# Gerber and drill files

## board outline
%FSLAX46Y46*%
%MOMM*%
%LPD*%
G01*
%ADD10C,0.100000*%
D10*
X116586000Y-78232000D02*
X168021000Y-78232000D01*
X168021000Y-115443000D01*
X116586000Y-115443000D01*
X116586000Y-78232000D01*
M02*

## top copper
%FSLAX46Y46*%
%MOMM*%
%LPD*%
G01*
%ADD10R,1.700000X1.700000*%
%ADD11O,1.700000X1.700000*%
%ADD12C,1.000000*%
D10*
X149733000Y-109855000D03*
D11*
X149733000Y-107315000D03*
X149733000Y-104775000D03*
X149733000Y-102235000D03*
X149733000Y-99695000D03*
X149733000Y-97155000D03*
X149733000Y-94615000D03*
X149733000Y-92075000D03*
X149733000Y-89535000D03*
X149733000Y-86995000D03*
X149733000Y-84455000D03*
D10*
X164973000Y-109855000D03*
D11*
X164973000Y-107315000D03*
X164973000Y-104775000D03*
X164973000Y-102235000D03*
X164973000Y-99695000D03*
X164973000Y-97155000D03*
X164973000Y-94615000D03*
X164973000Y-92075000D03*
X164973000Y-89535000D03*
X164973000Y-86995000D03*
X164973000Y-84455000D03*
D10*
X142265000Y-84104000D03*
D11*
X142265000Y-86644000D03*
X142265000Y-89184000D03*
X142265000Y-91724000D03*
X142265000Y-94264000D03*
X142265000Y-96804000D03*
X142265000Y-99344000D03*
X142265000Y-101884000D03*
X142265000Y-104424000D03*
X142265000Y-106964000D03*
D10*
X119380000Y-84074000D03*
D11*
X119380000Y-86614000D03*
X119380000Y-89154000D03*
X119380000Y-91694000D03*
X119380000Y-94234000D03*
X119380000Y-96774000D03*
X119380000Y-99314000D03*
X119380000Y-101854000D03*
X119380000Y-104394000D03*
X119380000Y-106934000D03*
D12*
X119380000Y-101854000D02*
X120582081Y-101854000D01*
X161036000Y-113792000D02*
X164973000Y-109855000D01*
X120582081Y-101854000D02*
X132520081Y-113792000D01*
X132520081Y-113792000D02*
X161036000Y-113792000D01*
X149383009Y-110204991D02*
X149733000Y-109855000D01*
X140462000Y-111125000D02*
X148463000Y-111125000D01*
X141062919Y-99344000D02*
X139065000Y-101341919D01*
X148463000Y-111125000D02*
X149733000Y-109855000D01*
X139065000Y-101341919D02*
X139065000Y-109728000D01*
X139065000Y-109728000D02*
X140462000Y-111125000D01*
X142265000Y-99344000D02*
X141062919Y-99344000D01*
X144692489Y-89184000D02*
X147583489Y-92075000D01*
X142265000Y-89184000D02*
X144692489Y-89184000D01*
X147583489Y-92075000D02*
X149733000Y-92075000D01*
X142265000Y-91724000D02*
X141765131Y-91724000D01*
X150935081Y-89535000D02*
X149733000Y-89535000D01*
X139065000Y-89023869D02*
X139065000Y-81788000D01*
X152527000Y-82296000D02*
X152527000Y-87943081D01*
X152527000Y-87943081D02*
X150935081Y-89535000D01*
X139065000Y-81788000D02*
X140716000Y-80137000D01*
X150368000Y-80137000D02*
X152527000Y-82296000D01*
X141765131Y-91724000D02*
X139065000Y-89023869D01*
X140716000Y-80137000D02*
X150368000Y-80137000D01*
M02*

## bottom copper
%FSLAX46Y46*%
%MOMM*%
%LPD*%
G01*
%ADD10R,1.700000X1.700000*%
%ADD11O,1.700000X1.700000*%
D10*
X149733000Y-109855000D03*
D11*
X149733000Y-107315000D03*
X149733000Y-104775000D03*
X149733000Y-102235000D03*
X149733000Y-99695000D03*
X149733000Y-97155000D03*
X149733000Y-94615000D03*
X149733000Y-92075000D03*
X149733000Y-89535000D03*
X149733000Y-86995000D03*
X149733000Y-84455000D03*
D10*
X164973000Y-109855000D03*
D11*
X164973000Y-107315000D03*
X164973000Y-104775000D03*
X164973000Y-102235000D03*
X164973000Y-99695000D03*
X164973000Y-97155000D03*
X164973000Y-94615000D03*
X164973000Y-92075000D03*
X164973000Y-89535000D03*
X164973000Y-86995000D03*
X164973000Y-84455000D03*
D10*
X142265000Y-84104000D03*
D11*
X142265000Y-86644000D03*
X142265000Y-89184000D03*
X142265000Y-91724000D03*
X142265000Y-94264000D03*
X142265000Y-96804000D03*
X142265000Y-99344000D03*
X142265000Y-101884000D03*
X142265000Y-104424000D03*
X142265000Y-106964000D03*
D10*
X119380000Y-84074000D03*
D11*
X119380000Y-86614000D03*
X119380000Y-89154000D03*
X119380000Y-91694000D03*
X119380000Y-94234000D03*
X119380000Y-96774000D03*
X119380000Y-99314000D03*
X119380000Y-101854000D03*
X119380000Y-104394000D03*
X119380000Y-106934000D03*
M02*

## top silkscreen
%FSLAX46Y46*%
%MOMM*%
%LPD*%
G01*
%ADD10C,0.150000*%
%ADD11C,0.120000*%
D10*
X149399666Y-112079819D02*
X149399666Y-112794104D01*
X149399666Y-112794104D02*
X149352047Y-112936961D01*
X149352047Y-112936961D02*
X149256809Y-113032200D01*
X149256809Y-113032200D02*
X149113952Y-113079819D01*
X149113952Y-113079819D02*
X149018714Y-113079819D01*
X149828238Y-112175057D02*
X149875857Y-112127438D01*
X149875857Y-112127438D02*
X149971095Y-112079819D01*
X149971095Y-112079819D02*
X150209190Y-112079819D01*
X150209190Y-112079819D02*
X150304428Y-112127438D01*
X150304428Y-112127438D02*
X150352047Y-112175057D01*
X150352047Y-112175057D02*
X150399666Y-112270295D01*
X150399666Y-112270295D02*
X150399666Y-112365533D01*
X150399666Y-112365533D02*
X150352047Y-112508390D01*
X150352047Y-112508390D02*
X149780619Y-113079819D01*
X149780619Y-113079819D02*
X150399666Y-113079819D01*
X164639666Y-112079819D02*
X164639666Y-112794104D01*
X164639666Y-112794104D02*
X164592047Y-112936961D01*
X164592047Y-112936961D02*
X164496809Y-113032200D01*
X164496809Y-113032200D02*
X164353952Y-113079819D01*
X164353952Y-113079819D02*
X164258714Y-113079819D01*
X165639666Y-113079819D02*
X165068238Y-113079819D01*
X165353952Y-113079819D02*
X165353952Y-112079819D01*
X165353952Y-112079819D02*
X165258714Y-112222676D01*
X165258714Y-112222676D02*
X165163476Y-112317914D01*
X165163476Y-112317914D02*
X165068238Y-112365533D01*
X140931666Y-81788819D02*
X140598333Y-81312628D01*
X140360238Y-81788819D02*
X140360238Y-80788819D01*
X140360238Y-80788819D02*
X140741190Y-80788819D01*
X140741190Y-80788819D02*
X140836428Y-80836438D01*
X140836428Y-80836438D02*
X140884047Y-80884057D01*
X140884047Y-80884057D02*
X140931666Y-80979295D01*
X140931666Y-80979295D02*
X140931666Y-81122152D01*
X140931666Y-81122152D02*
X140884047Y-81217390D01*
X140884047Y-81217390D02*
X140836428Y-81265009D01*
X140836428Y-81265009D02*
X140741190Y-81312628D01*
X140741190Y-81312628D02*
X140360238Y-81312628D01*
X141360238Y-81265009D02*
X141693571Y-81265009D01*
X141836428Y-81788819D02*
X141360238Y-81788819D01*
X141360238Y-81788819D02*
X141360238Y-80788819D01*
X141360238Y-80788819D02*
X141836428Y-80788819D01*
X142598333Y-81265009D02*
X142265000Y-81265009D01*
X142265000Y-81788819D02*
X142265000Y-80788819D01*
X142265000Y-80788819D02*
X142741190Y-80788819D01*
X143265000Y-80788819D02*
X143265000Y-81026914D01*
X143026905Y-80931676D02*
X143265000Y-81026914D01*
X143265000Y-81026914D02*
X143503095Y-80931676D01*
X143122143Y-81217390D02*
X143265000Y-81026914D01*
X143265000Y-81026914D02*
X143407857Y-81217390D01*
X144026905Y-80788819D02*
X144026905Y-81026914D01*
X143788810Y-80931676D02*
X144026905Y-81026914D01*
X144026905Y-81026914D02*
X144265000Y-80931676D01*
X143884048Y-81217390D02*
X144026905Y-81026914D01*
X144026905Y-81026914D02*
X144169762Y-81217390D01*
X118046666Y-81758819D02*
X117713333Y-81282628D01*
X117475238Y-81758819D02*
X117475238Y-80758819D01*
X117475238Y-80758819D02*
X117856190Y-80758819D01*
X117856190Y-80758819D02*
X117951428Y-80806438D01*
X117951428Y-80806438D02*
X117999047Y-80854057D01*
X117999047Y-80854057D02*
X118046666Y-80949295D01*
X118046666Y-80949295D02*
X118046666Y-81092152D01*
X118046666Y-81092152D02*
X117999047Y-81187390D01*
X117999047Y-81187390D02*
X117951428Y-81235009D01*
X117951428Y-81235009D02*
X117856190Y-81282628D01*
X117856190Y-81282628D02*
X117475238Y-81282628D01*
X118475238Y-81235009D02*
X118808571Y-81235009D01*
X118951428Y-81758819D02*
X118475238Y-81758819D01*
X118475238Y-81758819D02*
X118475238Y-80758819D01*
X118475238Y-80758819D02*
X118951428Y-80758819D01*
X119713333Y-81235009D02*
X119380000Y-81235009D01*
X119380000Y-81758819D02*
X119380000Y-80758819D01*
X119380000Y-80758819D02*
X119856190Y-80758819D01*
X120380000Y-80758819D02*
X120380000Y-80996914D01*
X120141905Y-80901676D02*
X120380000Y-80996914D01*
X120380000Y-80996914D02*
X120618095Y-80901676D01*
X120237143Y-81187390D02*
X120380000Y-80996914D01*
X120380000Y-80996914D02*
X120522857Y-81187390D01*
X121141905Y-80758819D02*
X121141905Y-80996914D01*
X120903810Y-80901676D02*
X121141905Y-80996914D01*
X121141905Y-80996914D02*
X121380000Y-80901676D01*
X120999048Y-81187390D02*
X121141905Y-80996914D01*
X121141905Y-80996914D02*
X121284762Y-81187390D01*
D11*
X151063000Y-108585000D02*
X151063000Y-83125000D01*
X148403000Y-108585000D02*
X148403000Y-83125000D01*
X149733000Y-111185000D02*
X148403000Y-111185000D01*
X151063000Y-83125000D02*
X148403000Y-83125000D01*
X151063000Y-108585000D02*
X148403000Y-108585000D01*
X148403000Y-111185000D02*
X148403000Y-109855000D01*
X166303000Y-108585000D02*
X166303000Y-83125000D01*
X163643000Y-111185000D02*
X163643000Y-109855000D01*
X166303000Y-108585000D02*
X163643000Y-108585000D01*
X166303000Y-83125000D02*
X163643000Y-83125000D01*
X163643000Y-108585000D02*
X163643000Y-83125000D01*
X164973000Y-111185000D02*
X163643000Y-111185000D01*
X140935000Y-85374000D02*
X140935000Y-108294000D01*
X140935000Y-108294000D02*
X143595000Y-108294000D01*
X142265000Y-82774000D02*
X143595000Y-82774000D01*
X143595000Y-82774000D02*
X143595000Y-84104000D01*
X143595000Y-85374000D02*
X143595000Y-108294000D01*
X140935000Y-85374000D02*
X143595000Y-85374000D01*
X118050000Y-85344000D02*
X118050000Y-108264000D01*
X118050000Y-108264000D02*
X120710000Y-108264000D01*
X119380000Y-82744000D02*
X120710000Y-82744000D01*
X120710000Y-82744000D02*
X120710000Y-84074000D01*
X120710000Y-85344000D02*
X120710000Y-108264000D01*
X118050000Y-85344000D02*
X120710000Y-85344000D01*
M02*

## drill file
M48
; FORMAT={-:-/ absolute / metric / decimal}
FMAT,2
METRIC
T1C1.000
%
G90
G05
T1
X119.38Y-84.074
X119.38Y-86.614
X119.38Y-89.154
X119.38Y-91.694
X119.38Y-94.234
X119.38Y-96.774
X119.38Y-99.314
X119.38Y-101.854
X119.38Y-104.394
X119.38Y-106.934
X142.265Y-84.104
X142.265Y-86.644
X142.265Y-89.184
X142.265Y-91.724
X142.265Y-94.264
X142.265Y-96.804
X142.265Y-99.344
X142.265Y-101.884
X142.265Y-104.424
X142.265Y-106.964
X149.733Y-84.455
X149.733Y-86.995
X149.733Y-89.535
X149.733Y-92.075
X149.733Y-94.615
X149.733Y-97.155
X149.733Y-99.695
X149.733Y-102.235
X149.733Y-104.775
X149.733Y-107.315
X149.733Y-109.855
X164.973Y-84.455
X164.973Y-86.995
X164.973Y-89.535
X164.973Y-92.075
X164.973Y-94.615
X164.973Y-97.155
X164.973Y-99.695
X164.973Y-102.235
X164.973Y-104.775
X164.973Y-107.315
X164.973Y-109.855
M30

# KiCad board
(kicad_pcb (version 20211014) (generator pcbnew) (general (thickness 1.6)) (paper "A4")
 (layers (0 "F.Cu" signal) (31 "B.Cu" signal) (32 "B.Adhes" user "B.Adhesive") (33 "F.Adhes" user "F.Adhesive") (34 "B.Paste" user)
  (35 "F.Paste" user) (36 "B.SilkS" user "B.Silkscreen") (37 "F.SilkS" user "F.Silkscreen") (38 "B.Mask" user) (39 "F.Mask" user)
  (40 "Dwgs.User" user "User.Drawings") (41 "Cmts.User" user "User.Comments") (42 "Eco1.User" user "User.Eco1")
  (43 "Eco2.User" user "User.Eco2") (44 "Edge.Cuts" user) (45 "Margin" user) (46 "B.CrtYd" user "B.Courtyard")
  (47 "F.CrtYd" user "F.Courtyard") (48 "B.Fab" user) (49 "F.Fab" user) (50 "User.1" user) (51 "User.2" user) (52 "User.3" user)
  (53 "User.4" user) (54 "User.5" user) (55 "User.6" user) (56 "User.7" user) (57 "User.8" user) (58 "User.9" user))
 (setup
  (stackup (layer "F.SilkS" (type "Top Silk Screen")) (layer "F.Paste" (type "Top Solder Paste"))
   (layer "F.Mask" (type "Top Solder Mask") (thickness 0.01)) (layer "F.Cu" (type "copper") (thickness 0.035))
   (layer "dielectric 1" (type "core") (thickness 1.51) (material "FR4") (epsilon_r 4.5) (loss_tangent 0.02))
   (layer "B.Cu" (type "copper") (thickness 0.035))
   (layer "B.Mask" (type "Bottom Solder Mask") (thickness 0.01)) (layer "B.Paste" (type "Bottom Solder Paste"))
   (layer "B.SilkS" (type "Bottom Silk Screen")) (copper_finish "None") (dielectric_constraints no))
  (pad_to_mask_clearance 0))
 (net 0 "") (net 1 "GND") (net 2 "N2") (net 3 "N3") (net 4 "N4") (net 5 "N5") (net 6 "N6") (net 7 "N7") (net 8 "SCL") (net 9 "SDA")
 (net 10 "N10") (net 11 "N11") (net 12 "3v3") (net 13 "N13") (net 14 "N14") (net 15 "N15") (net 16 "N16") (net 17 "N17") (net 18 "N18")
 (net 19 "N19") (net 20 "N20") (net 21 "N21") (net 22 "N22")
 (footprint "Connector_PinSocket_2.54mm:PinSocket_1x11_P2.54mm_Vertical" (layer "F.Cu") (at 149.733 109.855 180)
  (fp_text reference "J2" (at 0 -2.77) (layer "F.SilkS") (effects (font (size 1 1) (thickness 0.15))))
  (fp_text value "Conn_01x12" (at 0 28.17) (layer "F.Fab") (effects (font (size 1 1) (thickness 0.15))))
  (fp_line (start -1.33 1.27) (end -1.33 26.73) (layer "F.SilkS") (width 0.12))
  (fp_line (start 1.33 1.27) (end 1.33 26.73) (layer "F.SilkS") (width 0.12))
  (fp_line (start 0 -1.33) (end 1.33 -1.33) (layer "F.SilkS") (width 0.12))
  (fp_line (start -1.33 26.73) (end 1.33 26.73) (layer "F.SilkS") (width 0.12))
  (fp_line (start -1.33 1.27) (end 1.33 1.27) (layer "F.SilkS") (width 0.12))
  (fp_line (start 1.33 -1.33) (end 1.33 0) (layer "F.SilkS") (width 0.12))
  (pad "1" thru_hole rect (at 0 0 180) (size 1.7 1.7) (drill 1) (layers *.Cu *.Mask) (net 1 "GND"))
  (pad "2" thru_hole oval (at 0 2.54 180) (size 1.7 1.7) (drill 1) (layers *.Cu *.Mask) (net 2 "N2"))
  (pad "3" thru_hole oval (at 0 5.08 180) (size 1.7 1.7) (drill 1) (layers *.Cu *.Mask) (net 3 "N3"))
  (pad "4" thru_hole oval (at 0 7.62 180) (size 1.7 1.7) (drill 1) (layers *.Cu *.Mask) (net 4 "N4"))
  (pad "5" thru_hole oval (at 0 10.16 180) (size 1.7 1.7) (drill 1) (layers *.Cu *.Mask) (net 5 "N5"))
  (pad "6" thru_hole oval (at 0 12.7 180) (size 1.7 1.7) (drill 1) (layers *.Cu *.Mask) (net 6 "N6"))
  (pad "7" thru_hole oval (at 0 15.24 180) (size 1.7 1.7) (drill 1) (layers *.Cu *.Mask) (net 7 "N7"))
  (pad "8" thru_hole oval (at 0 17.78 180) (size 1.7 1.7) (drill 1) (layers *.Cu *.Mask) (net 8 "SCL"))
  (pad "9" thru_hole oval (at 0 20.32 180) (size 1.7 1.7) (drill 1) (layers *.Cu *.Mask) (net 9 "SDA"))
  (pad "10" thru_hole oval (at 0 22.86 180) (size 1.7 1.7) (drill 1) (layers *.Cu *.Mask) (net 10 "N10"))
  (pad "11" thru_hole oval (at 0 25.4 180) (size 1.7 1.7) (drill 1) (layers *.Cu *.Mask) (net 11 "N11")))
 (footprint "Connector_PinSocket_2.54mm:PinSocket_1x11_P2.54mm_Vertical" (layer "F.Cu") (at 164.973 109.855 180)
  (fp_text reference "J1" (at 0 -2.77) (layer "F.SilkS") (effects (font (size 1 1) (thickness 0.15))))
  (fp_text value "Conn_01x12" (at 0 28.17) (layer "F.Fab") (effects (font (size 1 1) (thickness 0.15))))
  (fp_line (start -1.33 1.27) (end -1.33 26.73) (layer "F.SilkS") (width 0.12))
  (fp_line (start 1.33 -1.33) (end 1.33 0) (layer "F.SilkS") (width 0.12))
  (fp_line (start -1.33 1.27) (end 1.33 1.27) (layer "F.SilkS") (width 0.12))
  (fp_line (start -1.33 26.73) (end 1.33 26.73) (layer "F.SilkS") (width 0.12))
  (fp_line (start 1.33 1.27) (end 1.33 26.73) (layer "F.SilkS") (width 0.12))
  (fp_line (start 0 -1.33) (end 1.33 -1.33) (layer "F.SilkS") (width 0.12))
  (pad "1" thru_hole rect (at 0 0 180) (size 1.7 1.7) (drill 1) (layers *.Cu *.Mask) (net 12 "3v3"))
  (pad "2" thru_hole oval (at 0 2.54 180) (size 1.7 1.7) (drill 1) (layers *.Cu *.Mask) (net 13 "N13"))
  (pad "3" thru_hole oval (at 0 5.08 180) (size 1.7 1.7) (drill 1) (layers *.Cu *.Mask) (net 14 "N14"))
  (pad "4" thru_hole oval (at 0 7.62 180) (size 1.7 1.7) (drill 1) (layers *.Cu *.Mask) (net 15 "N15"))
  (pad "5" thru_hole oval (at 0 10.16 180) (size 1.7 1.7) (drill 1) (layers *.Cu *.Mask) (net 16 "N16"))
  (pad "6" thru_hole oval (at 0 12.7 180) (size 1.7 1.7) (drill 1) (layers *.Cu *.Mask) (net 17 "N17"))
  (pad "7" thru_hole oval (at 0 15.24 180) (size 1.7 1.7) (drill 1) (layers *.Cu *.Mask) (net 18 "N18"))
  (pad "8" thru_hole oval (at 0 17.78 180) (size 1.7 1.7) (drill 1) (layers *.Cu *.Mask) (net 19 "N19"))
  (pad "9" thru_hole oval (at 0 20.32 180) (size 1.7 1.7) (drill 1) (layers *.Cu *.Mask) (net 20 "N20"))
  (pad "10" thru_hole oval (at 0 22.86 180) (size 1.7 1.7) (drill 1) (layers *.Cu *.Mask) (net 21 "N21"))
  (pad "11" thru_hole oval (at 0 25.4 180) (size 1.7 1.7) (drill 1) (layers *.Cu *.Mask) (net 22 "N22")))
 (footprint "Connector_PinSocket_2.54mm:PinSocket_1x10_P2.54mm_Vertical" (layer "F.Cu") (at 142.265 84.104)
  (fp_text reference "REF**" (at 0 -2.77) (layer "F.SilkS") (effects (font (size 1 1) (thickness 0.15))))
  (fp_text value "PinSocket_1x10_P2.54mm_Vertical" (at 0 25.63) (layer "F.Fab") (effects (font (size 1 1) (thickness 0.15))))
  (fp_line (start -1.33 1.27) (end -1.33 24.19) (layer "F.SilkS") (width 0.12))
  (fp_line (start -1.33 24.19) (end 1.33 24.19) (layer "F.SilkS") (width 0.12))
  (fp_line (start 0 -1.33) (end 1.33 -1.33) (layer "F.SilkS") (width 0.12))
  (fp_line (start 1.33 -1.33) (end 1.33 0) (layer "F.SilkS") (width 0.12))
  (fp_line (start 1.33 1.27) (end 1.33 24.19) (layer "F.SilkS") (width 0.12))
  (fp_line (start -1.33 1.27) (end 1.33 1.27) (layer "F.SilkS") (width 0.12))
  (pad "1" thru_hole rect (at 0 0) (size 1.7 1.7) (drill 1) (layers *.Cu *.Mask))
  (pad "2" thru_hole oval (at 0 2.54) (size 1.7 1.7) (drill 1) (layers *.Cu *.Mask))
  (pad "3" thru_hole oval (at 0 5.08) (size 1.7 1.7) (drill 1) (layers *.Cu *.Mask) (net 8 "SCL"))
  (pad "4" thru_hole oval (at 0 7.62) (size 1.7 1.7) (drill 1) (layers *.Cu *.Mask) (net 9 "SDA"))
  (pad "5" thru_hole oval (at 0 10.16) (size 1.7 1.7) (drill 1) (layers *.Cu *.Mask))
  (pad "6" thru_hole oval (at 0 12.7) (size 1.7 1.7) (drill 1) (layers *.Cu *.Mask))
  (pad "7" thru_hole oval (at 0 15.24) (size 1.7 1.7) (drill 1) (layers *.Cu *.Mask) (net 1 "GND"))
  (pad "8" thru_hole oval (at 0 17.78) (size 1.7 1.7) (drill 1) (layers *.Cu *.Mask))
  (pad "9" thru_hole oval (at 0 20.32) (size 1.7 1.7) (drill 1) (layers *.Cu *.Mask))
  (pad "10" thru_hole oval (at 0 22.86) (size 1.7 1.7) (drill 1) (layers *.Cu *.Mask)))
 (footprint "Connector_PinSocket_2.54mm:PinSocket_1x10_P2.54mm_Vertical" (layer "F.Cu") (at 119.38 84.074)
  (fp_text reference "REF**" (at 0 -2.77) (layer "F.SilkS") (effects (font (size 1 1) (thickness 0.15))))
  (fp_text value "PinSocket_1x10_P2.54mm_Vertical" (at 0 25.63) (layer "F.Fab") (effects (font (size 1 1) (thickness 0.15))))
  (fp_line (start -1.33 1.27) (end -1.33 24.19) (layer "F.SilkS") (width 0.12))
  (fp_line (start -1.33 24.19) (end 1.33 24.19) (layer "F.SilkS") (width 0.12))
  (fp_line (start 0 -1.33) (end 1.33 -1.33) (layer "F.SilkS") (width 0.12))
  (fp_line (start 1.33 -1.33) (end 1.33 0) (layer "F.SilkS") (width 0.12))
  (fp_line (start 1.33 1.27) (end 1.33 24.19) (layer "F.SilkS") (width 0.12))
  (fp_line (start -1.33 1.27) (end 1.33 1.27) (layer "F.SilkS") (width 0.12))
  (pad "1" thru_hole rect (at 0 0) (size 1.7 1.7) (drill 1) (layers *.Cu *.Mask))
  (pad "2" thru_hole oval (at 0 2.54) (size 1.7 1.7) (drill 1) (layers *.Cu *.Mask))
  (pad "3" thru_hole oval (at 0 5.08) (size 1.7 1.7) (drill 1) (layers *.Cu *.Mask))
  (pad "4" thru_hole oval (at 0 7.62) (size 1.7 1.7) (drill 1) (layers *.Cu *.Mask))
  (pad "5" thru_hole oval (at 0 10.16) (size 1.7 1.7) (drill 1) (layers *.Cu *.Mask))
  (pad "6" thru_hole oval (at 0 12.7) (size 1.7 1.7) (drill 1) (layers *.Cu *.Mask))
  (pad "7" thru_hole oval (at 0 15.24) (size 1.7 1.7) (drill 1) (layers *.Cu *.Mask))
  (pad "8" thru_hole oval (at 0 17.78) (size 1.7 1.7) (drill 1) (layers *.Cu *.Mask) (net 12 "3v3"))
  (pad "9" thru_hole oval (at 0 20.32) (size 1.7 1.7) (drill 1) (layers *.Cu *.Mask))
  (pad "10" thru_hole oval (at 0 22.86) (size 1.7 1.7) (drill 1) (layers *.Cu *.Mask)))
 (gr_rect (start 116.586 78.232) (end 168.021 115.443) (layer "Edge.Cuts") (width 0.1) (fill none))
 (segment (start 119.38 101.854) (end 120.582081 101.854) (width 1) (layer "F.Cu") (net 12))
 (segment (start 161.036 113.792) (end 164.973 109.855) (width 1) (layer "F.Cu") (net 12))
 (segment (start 120.582081 101.854) (end 132.520081 113.792) (width 1) (layer "F.Cu") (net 12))
 (segment (start 132.520081 113.792) (end 161.036 113.792) (width 1) (layer "F.Cu") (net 12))
 (segment (start 149.383009 110.204991) (end 149.733 109.855) (width 1) (layer "F.Cu") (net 1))
 (segment (start 140.462 111.125) (end 148.463 111.125) (width 1) (layer "F.Cu") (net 1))
 (segment (start 141.062919 99.344) (end 139.065 101.341919) (width 1) (layer "F.Cu") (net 1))
 (segment (start 148.463 111.125) (end 149.733 109.855) (width 1) (layer "F.Cu") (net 1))
 (segment (start 139.065 101.341919) (end 139.065 109.728) (width 1) (layer "F.Cu") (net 1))
 (segment (start 139.065 109.728) (end 140.462 111.125) (width 1) (layer "F.Cu") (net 1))
 (segment (start 142.265 99.344) (end 141.062919 99.344) (width 1) (layer "F.Cu") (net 1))
 (segment (start 144.692489 89.184) (end 147.583489 92.075) (width 1) (layer "F.Cu") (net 8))
 (segment (start 142.265 89.184) (end 144.692489 89.184) (width 1) (layer "F.Cu") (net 8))
 (segment (start 147.583489 92.075) (end 149.733 92.075) (width 1) (layer "F.Cu") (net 8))
 (segment (start 142.265 91.724) (end 141.765131 91.724) (width 1) (layer "F.Cu") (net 9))
 (segment (start 150.935081 89.535) (end 149.733 89.535) (width 1) (layer "F.Cu") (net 9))
 (segment (start 139.065 89.023869) (end 139.065 81.788) (width 1) (layer "F.Cu") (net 9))
 (segment (start 152.527 82.296) (end 152.527 87.943081) (width 1) (layer "F.Cu") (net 9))
 (segment (start 152.527 87.943081) (end 150.935081 89.535) (width 1) (layer "F.Cu") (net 9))
 (segment (start 139.065 81.788) (end 140.716 80.137) (width 1) (layer "F.Cu") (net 9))
 (segment (start 150.368 80.137) (end 152.527 82.296) (width 1) (layer "F.Cu") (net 9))
 (segment (start 141.765131 91.724) (end 139.065 89.023869) (width 1) (layer "F.Cu") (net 9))
 (segment (start 140.716 80.137) (end 150.368 80.137) (width 1) (layer "F.Cu") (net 9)))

